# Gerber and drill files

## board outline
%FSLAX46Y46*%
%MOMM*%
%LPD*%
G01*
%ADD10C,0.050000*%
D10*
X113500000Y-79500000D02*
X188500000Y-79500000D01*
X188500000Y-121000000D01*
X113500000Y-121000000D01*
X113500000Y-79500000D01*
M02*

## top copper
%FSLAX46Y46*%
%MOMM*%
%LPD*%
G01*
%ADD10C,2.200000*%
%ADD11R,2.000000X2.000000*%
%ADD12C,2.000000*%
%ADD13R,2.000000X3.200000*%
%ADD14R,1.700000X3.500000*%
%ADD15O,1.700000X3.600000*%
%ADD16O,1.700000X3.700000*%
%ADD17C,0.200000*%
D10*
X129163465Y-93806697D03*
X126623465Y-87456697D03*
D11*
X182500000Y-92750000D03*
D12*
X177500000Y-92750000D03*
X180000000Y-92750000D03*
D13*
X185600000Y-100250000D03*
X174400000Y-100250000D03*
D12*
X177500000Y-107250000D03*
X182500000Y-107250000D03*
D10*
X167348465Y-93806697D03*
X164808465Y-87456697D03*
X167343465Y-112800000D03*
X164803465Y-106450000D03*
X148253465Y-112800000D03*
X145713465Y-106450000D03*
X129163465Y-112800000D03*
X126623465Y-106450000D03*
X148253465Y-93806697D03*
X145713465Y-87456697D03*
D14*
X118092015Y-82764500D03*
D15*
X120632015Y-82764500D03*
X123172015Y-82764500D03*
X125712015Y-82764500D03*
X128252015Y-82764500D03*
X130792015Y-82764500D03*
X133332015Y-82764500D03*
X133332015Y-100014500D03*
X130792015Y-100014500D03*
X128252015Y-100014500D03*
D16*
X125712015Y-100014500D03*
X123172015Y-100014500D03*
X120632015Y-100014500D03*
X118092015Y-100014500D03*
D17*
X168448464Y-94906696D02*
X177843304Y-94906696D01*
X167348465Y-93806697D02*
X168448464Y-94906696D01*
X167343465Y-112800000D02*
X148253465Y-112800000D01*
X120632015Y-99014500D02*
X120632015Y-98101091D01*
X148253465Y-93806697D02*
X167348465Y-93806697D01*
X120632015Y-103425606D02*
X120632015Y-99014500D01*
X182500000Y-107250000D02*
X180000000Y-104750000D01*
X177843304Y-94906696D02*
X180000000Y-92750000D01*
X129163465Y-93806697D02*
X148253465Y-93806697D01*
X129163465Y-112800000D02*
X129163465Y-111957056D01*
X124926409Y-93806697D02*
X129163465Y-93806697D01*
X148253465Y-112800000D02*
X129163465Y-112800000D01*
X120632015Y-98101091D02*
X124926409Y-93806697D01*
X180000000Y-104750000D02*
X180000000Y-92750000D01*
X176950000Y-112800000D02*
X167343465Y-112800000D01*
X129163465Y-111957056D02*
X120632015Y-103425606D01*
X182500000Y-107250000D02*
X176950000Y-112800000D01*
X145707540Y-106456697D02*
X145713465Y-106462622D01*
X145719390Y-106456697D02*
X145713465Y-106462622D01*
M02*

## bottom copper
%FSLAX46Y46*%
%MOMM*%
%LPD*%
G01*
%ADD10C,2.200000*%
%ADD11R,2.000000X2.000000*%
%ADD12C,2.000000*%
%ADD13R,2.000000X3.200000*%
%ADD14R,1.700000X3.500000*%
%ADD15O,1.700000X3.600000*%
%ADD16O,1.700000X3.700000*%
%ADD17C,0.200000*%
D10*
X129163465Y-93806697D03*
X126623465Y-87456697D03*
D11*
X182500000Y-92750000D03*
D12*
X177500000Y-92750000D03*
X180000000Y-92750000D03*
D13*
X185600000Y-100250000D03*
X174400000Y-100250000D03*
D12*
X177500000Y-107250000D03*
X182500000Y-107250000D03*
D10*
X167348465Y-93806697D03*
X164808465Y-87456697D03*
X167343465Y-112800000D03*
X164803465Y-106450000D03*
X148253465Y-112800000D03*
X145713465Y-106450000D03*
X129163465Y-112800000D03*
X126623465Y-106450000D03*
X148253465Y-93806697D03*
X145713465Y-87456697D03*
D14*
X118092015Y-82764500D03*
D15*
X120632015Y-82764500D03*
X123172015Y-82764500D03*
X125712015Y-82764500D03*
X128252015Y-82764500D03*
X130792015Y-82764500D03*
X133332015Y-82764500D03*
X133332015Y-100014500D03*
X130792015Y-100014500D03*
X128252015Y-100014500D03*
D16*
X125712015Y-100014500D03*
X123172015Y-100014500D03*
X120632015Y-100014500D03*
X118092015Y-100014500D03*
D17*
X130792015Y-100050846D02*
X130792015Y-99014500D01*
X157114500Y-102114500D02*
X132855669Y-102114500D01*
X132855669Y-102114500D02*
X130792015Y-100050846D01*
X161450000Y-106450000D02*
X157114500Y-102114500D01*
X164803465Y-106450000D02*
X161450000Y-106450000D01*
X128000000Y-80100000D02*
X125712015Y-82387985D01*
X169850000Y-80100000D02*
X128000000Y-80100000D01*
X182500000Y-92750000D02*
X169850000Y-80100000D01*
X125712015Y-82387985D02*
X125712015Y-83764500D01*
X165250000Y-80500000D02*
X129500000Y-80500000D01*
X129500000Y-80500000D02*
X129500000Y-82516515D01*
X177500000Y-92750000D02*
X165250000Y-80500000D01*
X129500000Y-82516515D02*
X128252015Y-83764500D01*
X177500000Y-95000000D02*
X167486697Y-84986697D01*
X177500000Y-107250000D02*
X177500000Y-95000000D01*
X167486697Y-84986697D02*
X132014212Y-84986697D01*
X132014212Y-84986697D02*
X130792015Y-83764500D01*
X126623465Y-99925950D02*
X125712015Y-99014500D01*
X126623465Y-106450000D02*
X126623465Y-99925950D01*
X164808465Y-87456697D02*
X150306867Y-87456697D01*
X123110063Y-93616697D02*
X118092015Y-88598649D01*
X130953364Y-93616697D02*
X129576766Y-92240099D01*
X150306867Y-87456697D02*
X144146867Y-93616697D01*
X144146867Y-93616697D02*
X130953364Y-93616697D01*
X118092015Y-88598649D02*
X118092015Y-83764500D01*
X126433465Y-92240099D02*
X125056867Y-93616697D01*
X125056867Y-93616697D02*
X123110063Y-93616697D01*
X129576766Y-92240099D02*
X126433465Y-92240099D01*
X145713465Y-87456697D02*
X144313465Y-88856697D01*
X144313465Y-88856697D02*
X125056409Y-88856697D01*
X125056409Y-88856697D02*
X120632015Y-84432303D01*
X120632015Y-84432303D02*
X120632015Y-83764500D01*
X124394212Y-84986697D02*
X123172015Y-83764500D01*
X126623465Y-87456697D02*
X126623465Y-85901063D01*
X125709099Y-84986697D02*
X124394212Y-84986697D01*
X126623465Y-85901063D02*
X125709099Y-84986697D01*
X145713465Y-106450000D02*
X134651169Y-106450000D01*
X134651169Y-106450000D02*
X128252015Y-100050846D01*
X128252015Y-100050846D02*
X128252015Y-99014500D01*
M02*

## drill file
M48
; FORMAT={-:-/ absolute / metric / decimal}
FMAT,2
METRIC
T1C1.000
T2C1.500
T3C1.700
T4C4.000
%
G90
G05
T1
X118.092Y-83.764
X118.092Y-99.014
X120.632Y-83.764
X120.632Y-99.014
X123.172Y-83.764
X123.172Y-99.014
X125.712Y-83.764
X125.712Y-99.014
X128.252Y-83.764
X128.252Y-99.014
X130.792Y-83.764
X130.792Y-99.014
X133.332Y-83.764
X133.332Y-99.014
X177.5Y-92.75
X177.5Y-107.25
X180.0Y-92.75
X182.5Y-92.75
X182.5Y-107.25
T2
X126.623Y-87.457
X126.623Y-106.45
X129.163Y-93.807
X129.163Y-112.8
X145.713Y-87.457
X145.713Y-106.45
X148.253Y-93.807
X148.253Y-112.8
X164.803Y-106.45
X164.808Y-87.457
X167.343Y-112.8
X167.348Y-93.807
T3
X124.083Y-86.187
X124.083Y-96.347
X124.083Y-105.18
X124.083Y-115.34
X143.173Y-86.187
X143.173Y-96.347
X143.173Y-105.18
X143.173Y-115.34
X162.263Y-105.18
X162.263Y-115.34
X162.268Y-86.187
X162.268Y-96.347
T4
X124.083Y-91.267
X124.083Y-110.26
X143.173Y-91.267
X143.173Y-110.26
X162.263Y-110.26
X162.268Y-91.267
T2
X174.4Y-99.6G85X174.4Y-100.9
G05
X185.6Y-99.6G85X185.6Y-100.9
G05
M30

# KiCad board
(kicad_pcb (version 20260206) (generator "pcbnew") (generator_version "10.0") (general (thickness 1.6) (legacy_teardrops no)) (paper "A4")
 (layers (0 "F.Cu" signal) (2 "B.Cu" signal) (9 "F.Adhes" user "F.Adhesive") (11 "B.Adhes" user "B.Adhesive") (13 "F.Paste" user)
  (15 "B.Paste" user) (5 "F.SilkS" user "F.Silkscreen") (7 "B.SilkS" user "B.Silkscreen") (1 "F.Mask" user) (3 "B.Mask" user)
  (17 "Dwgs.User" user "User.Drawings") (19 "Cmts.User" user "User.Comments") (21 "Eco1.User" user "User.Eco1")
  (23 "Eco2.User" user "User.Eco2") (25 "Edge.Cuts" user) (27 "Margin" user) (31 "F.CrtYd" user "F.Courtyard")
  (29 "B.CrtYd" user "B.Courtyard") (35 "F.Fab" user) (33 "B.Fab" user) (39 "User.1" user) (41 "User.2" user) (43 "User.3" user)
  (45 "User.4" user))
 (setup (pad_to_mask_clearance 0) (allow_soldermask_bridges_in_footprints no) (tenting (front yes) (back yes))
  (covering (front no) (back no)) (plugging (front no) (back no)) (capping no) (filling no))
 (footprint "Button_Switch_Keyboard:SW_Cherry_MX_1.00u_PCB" (layer "F.Cu") (at 129.163465 93.806697 -90)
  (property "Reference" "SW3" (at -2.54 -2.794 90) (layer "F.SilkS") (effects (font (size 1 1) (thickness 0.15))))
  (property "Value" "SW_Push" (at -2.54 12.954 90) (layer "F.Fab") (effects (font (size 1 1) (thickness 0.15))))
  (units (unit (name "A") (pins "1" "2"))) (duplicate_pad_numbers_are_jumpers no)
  (pad "" np_thru_hole circle (at -7.62 5.08 270) (size 1.7 1.7) (drill 1.7) (layers "*.Cu" "*.Mask"))
  (pad "" np_thru_hole circle (at -2.54 5.08 270) (size 4 4) (drill 4) (layers "*.Cu" "*.Mask"))
  (pad "" np_thru_hole circle (at 2.54 5.08 270) (size 1.7 1.7) (drill 1.7) (layers "*.Cu" "*.Mask"))
  (pad "1" thru_hole circle (at 0 0 270) (size 2.2 2.2) (drill 1.5) (layers "*.Cu" "*.Mask") (remove_unused_layers no) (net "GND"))
  (pad "2" thru_hole circle (at -6.35 2.54 270) (size 2.2 2.2) (drill 1.5) (layers "*.Cu" "*.Mask") (remove_unused_layers no)
   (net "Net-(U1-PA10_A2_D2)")))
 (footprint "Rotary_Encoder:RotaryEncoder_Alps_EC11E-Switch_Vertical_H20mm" (layer "F.Cu") (at 182.5 92.75 -90)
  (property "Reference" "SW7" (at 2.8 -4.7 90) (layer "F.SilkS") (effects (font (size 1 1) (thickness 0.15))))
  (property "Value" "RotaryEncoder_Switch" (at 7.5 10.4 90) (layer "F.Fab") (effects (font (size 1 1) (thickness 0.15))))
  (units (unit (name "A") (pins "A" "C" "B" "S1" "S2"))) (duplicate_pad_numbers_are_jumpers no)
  (pad "A" thru_hole rect (at 0 0 270) (size 2 2) (drill 1) (layers "*.Cu" "*.Mask") (remove_unused_layers no) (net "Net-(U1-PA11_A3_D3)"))
  (pad "B" thru_hole circle (at 0 5 270) (size 2 2) (drill 1) (layers "*.Cu" "*.Mask") (remove_unused_layers no)
   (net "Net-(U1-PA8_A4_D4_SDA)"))
  (pad "C" thru_hole circle (at 0 2.5 270) (size 2 2) (drill 1) (layers "*.Cu" "*.Mask") (remove_unused_layers no) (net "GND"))
  (pad "MP" thru_hole rect (at 7.5 -3.1 270) (size 3.2 2) (drill oval 2.8 1.5) (layers "*.Cu" "*.Mask") (remove_unused_layers no))
  (pad "MP" thru_hole rect (at 7.5 8.1 270) (size 3.2 2) (drill oval 2.8 1.5) (layers "*.Cu" "*.Mask") (remove_unused_layers no))
  (pad "S1" thru_hole circle (at 14.5 5 270) (size 2 2) (drill 1) (layers "*.Cu" "*.Mask") (remove_unused_layers no)
   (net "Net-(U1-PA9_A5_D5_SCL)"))
  (pad "S2" thru_hole circle (at 14.5 0 270) (size 2 2) (drill 1) (layers "*.Cu" "*.Mask") (remove_unused_layers no) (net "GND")))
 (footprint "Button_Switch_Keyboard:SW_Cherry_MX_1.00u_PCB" (layer "F.Cu") (at 167.348465 93.806697 -90)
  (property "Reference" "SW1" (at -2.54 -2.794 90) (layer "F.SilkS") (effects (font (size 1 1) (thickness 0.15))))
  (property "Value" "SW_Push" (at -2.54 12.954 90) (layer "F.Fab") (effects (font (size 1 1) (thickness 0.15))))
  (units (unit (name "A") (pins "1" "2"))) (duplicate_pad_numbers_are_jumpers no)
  (pad "" np_thru_hole circle (at -7.62 5.08 270) (size 1.7 1.7) (drill 1.7) (layers "*.Cu" "*.Mask"))
  (pad "" np_thru_hole circle (at -2.54 5.08 270) (size 4 4) (drill 4) (layers "*.Cu" "*.Mask"))
  (pad "" np_thru_hole circle (at 2.54 5.08 270) (size 1.7 1.7) (drill 1.7) (layers "*.Cu" "*.Mask"))
  (pad "1" thru_hole circle (at 0 0 270) (size 2.2 2.2) (drill 1.5) (layers "*.Cu" "*.Mask") (remove_unused_layers no) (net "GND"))
  (pad "2" thru_hole circle (at -6.35 2.54 270) (size 2.2 2.2) (drill 1.5) (layers "*.Cu" "*.Mask") (remove_unused_layers no)
   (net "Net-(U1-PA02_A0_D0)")))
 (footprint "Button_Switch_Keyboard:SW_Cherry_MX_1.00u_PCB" (layer "F.Cu") (at 167.343465 112.8 -90)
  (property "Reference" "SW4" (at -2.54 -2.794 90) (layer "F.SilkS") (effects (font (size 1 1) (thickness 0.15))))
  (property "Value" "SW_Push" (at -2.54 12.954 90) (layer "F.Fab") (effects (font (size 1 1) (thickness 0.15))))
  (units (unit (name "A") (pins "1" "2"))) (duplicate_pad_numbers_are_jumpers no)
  (pad "" np_thru_hole circle (at -7.62 5.08 270) (size 1.7 1.7) (drill 1.7) (layers "*.Cu" "*.Mask"))
  (pad "" np_thru_hole circle (at -2.54 5.08 270) (size 4 4) (drill 4) (layers "*.Cu" "*.Mask"))
  (pad "" np_thru_hole circle (at 2.54 5.08 270) (size 1.7 1.7) (drill 1.7) (layers "*.Cu" "*.Mask"))
  (pad "1" thru_hole circle (at 0 0 270) (size 2.2 2.2) (drill 1.5) (layers "*.Cu" "*.Mask") (remove_unused_layers no) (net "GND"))
  (pad "2" thru_hole circle (at -6.35 2.54 270) (size 2.2 2.2) (drill 1.5) (layers "*.Cu" "*.Mask") (remove_unused_layers no)
   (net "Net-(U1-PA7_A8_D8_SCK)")))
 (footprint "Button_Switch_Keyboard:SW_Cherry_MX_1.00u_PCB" (layer "F.Cu") (at 148.253465 112.8 -90)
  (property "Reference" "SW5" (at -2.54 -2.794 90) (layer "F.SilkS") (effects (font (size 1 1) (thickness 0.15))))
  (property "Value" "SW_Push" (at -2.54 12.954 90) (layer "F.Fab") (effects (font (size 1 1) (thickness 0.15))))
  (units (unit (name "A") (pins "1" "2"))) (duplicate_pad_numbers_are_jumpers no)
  (pad "" np_thru_hole circle (at -7.62 5.08 270) (size 1.7 1.7) (drill 1.7) (layers "*.Cu" "*.Mask"))
  (pad "" np_thru_hole circle (at -2.54 5.08 270) (size 4 4) (drill 4) (layers "*.Cu" "*.Mask"))
  (pad "" np_thru_hole circle (at 2.54 5.08 270) (size 1.7 1.7) (drill 1.7) (layers "*.Cu" "*.Mask"))
  (pad "1" thru_hole circle (at 0 0 270) (size 2.2 2.2) (drill 1.5) (layers "*.Cu" "*.Mask") (remove_unused_layers no) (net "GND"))
  (pad "2" thru_hole circle (at -6.35 2.54 270) (size 2.2 2.2) (drill 1.5) (layers "*.Cu" "*.Mask") (remove_unused_layers no)
   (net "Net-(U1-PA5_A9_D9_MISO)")))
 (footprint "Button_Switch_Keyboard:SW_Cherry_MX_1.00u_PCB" (layer "F.Cu") (at 129.163465 112.8 -90)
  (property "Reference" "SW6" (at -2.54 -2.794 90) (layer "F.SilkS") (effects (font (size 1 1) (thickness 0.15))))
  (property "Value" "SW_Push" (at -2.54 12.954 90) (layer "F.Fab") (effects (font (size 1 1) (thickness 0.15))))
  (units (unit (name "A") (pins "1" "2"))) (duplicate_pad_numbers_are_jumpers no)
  (pad "" np_thru_hole circle (at -7.62 5.08 270) (size 1.7 1.7) (drill 1.7) (layers "*.Cu" "*.Mask"))
  (pad "" np_thru_hole circle (at -2.54 5.08 270) (size 4 4) (drill 4) (layers "*.Cu" "*.Mask"))
  (pad "" np_thru_hole circle (at 2.54 5.08 270) (size 1.7 1.7) (drill 1.7) (layers "*.Cu" "*.Mask"))
  (pad "1" thru_hole circle (at 0 0 270) (size 2.2 2.2) (drill 1.5) (layers "*.Cu" "*.Mask") (remove_unused_layers no) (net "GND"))
  (pad "2" thru_hole circle (at -6.35 2.54 270) (size 2.2 2.2) (drill 1.5) (layers "*.Cu" "*.Mask") (remove_unused_layers no)
   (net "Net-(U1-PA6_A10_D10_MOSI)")))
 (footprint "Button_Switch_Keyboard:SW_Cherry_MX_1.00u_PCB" (layer "F.Cu") (at 148.253465 93.806697 -90)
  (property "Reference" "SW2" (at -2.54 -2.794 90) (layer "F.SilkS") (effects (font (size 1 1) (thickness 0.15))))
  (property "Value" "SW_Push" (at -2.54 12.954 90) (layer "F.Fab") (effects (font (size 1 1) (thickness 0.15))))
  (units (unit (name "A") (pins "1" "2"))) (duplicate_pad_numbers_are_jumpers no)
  (pad "" np_thru_hole circle (at -7.62 5.08 270) (size 1.7 1.7) (drill 1.7) (layers "*.Cu" "*.Mask"))
  (pad "" np_thru_hole circle (at -2.54 5.08 270) (size 4 4) (drill 4) (layers "*.Cu" "*.Mask"))
  (pad "" np_thru_hole circle (at 2.54 5.08 270) (size 1.7 1.7) (drill 1.7) (layers "*.Cu" "*.Mask"))
  (pad "1" thru_hole circle (at 0 0 270) (size 2.2 2.2) (drill 1.5) (layers "*.Cu" "*.Mask") (remove_unused_layers no) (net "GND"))
  (pad "2" thru_hole circle (at -6.35 2.54 270) (size 2.2 2.2) (drill 1.5) (layers "*.Cu" "*.Mask") (remove_unused_layers no)
   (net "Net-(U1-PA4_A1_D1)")))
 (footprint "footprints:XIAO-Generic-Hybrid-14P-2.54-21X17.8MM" (layer "B.Cu") (at 125.712015 91.3895 -90)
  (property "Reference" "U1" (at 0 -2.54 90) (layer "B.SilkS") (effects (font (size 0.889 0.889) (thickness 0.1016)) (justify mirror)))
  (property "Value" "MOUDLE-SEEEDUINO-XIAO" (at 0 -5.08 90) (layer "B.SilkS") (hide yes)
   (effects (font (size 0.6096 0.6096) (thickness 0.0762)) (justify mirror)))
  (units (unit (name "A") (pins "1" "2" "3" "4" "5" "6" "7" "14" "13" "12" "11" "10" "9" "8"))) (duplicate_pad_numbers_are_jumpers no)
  (pad "1" thru_hole rect (at -7.625 7.62 270) (size 3.5 1.7) (drill 1 (offset -1 0)) (layers "*.Cu" "*.Mask") (remove_unused_layers no)
   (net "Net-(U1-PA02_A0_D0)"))
  (pad "2" thru_hole oval (at -7.625 5.08 270) (size 3.6 1.7) (drill 1 (offset -1 0)) (layers "*.Cu" "*.Mask") (remove_unused_layers no)
   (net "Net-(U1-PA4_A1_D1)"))
  (pad "3" thru_hole oval (at -7.625 2.54 270) (size 3.6 1.7) (drill 1 (offset -1 0)) (layers "*.Cu" "*.Mask") (remove_unused_layers no)
   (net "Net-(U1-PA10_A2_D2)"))
  (pad "4" thru_hole oval (at -7.625 0 270) (size 3.6 1.7) (drill 1 (offset -1 0)) (layers "*.Cu" "*.Mask") (remove_unused_layers no)
   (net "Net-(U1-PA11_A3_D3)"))
  (pad "5" thru_hole oval (at -7.625 -2.54 270) (size 3.6 1.7) (drill 1 (offset -1 0)) (layers "*.Cu" "*.Mask") (remove_unused_layers no)
   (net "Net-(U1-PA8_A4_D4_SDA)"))
  (pad "6" thru_hole oval (at -7.625 -5.08 90) (size 3.6 1.7) (drill 1 (offset 1 0)) (layers "*.Cu" "*.Mask") (remove_unused_layers no)
   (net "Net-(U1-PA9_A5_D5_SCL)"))
  (pad "7" thru_hole oval (at -7.625 -7.62 270) (size 3.6 1.7) (drill 1 (offset -1 0)) (layers "*.Cu" "*.Mask") (remove_unused_layers no)
   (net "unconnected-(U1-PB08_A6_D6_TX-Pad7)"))
  (pad "8" thru_hole oval (at 7.625 -7.62 270) (size 3.6 1.7) (drill 1 (offset 1 0)) (layers "*.Cu" "*.Mask") (remove_unused_layers no)
   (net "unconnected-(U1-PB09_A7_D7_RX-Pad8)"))
  (pad "9" thru_hole oval (at 7.625 -5.08 270) (size 3.6 1.7) (drill 1 (offset 1 0)) (layers "*.Cu" "*.Mask") (remove_unused_layers no)
   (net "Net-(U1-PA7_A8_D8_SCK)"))
  (pad "10" thru_hole oval (at 7.625 -2.54 270) (size 3.6 1.7) (drill 1 (offset 1 0)) (layers "*.Cu" "*.Mask") (remove_unused_layers no)
   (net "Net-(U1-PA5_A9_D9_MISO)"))
  (pad "11" thru_hole oval (at 7.625 0 270) (size 3.7 1.7) (drill 1 (offset 1 0)) (layers "*.Cu" "*.Mask") (remove_unused_layers no)
   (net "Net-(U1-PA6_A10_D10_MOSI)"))
  (pad "12" thru_hole oval (at 7.625 2.54 270) (size 3.7 1.7) (drill 1 (offset 1 0)) (layers "*.Cu" "*.Mask") (remove_unused_layers no)
   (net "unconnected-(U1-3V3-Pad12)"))
  (pad "13" thru_hole oval (at 7.625 5.08 270) (size 3.7 1.7) (drill 1 (offset 1 0)) (layers "*.Cu" "*.Mask") (remove_unused_layers no)
   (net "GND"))
  (pad "14" thru_hole oval (at 7.625 7.62 270) (size 3.7 1.7) (drill 1 (offset 1 0)) (layers "*.Cu" "*.Mask") (remove_unused_layers no)
   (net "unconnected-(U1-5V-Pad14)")))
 (gr_rect (start 113.5 79.5) (end 188.5 121) (stroke (width 0.05) (type default)) (fill no) (layer "Edge.Cuts"))
 (segment (start 130.792015 100.050846) (end 130.792015 99.0145) (width 0.2) (layer "B.Cu") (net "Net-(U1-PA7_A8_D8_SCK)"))
 (segment (start 157.1145 102.1145) (end 132.855669 102.1145) (width 0.2) (layer "B.Cu") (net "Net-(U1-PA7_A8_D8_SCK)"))
 (segment (start 132.855669 102.1145) (end 130.792015 100.050846) (width 0.2) (layer "B.Cu") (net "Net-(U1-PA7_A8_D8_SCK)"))
 (segment (start 161.45 106.45) (end 157.1145 102.1145) (width 0.2) (layer "B.Cu") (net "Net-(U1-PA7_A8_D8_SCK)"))
 (segment (start 164.803465 106.45) (end 161.45 106.45) (width 0.2) (layer "B.Cu") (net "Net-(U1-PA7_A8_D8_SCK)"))
 (segment (start 168.448464 94.906696) (end 177.843304 94.906696) (width 0.2) (layer "F.Cu") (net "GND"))
 (segment (start 167.348465 93.806697) (end 168.448464 94.906696) (width 0.2) (layer "F.Cu") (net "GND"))
 (segment (start 167.343465 112.8) (end 148.253465 112.8) (width 0.2) (layer "F.Cu") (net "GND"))
 (segment (start 120.632015 99.0145) (end 120.632015 98.101091) (width 0.2) (layer "F.Cu") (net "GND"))
 (segment (start 148.253465 93.806697) (end 167.348465 93.806697) (width 0.2) (layer "F.Cu") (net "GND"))
 (segment (start 120.632015 103.425606) (end 120.632015 99.0145) (width 0.2) (layer "F.Cu") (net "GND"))
 (segment (start 182.5 107.25) (end 180 104.75) (width 0.2) (layer "F.Cu") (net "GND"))
 (segment (start 177.843304 94.906696) (end 180 92.75) (width 0.2) (layer "F.Cu") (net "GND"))
 (segment (start 129.163465 93.806697) (end 148.253465 93.806697) (width 0.2) (layer "F.Cu") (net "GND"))
 (segment (start 129.163465 112.8) (end 129.163465 111.957056) (width 0.2) (layer "F.Cu") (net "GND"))
 (segment (start 124.926409 93.806697) (end 129.163465 93.806697) (width 0.2) (layer "F.Cu") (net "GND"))
 (segment (start 148.253465 112.8) (end 129.163465 112.8) (width 0.2) (layer "F.Cu") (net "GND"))
 (segment (start 120.632015 98.101091) (end 124.926409 93.806697) (width 0.2) (layer "F.Cu") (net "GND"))
 (segment (start 180 104.75) (end 180 92.75) (width 0.2) (layer "F.Cu") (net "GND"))
 (segment (start 176.95 112.8) (end 167.343465 112.8) (width 0.2) (layer "F.Cu") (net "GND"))
 (segment (start 129.163465 111.957056) (end 120.632015 103.425606) (width 0.2) (layer "F.Cu") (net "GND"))
 (segment (start 182.5 107.25) (end 176.95 112.8) (width 0.2) (layer "F.Cu") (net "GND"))
 (segment (start 128 80.1) (end 125.712015 82.387985) (width 0.2) (layer "B.Cu") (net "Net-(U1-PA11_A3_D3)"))
 (segment (start 169.85 80.1) (end 128 80.1) (width 0.2) (layer "B.Cu") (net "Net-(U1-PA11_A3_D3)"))
 (segment (start 182.5 92.75) (end 169.85 80.1) (width 0.2) (layer "B.Cu") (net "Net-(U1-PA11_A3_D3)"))
 (segment (start 125.712015 82.387985) (end 125.712015 83.7645) (width 0.2) (layer "B.Cu") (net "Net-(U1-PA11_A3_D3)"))
 (segment (start 165.25 80.5) (end 129.5 80.5) (width 0.2) (layer "B.Cu") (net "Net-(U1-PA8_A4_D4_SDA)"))
 (segment (start 129.5 80.5) (end 129.5 82.516515) (width 0.2) (layer "B.Cu") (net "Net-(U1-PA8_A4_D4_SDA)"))
 (segment (start 177.5 92.75) (end 165.25 80.5) (width 0.2) (layer "B.Cu") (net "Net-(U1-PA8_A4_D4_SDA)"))
 (segment (start 129.5 82.516515) (end 128.252015 83.7645) (width 0.2) (layer "B.Cu") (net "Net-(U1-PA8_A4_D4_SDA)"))
 (segment (start 177.5 95) (end 167.486697 84.986697) (width 0.2) (layer "B.Cu") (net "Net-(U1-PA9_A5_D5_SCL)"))
 (segment (start 177.5 107.25) (end 177.5 95) (width 0.2) (layer "B.Cu") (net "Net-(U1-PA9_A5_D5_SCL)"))
 (segment (start 167.486697 84.986697) (end 132.014212 84.986697) (width 0.2) (layer "B.Cu") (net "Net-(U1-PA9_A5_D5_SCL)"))
 (segment (start 132.014212 84.986697) (end 130.792015 83.7645) (width 0.2) (layer "B.Cu") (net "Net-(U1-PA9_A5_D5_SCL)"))
 (segment (start 126.623465 99.92595) (end 125.712015 99.0145) (width 0.2) (layer "B.Cu") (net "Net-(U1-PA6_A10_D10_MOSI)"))
 (segment (start 126.623465 106.45) (end 126.623465 99.92595) (width 0.2) (layer "B.Cu") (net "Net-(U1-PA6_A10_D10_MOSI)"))
 (segment (start 164.808465 87.456697) (end 150.306867 87.456697) (width 0.2) (layer "B.Cu") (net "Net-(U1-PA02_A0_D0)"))
 (segment (start 123.110063 93.616697) (end 118.092015 88.598649) (width 0.2) (layer "B.Cu") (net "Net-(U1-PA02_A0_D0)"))
 (segment (start 130.953364 93.616697) (end 129.576766 92.240099) (width 0.2) (layer "B.Cu") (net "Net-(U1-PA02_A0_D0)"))
 (segment (start 150.306867 87.456697) (end 144.146867 93.616697) (width 0.2) (layer "B.Cu") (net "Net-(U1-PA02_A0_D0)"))
 (segment (start 144.146867 93.616697) (end 130.953364 93.616697) (width 0.2) (layer "B.Cu") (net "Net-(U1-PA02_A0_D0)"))
 (segment (start 118.092015 88.598649) (end 118.092015 83.7645) (width 0.2) (layer "B.Cu") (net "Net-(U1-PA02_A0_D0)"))
 (segment (start 126.433465 92.240099) (end 125.056867 93.616697) (width 0.2) (layer "B.Cu") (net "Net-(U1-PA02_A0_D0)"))
 (segment (start 125.056867 93.616697) (end 123.110063 93.616697) (width 0.2) (layer "B.Cu") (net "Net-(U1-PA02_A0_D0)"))
 (segment (start 129.576766 92.240099) (end 126.433465 92.240099) (width 0.2) (layer "B.Cu") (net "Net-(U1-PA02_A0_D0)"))
 (segment (start 145.713465 87.456697) (end 144.313465 88.856697) (width 0.2) (layer "B.Cu") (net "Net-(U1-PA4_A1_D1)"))
 (segment (start 144.313465 88.856697) (end 125.056409 88.856697) (width 0.2) (layer "B.Cu") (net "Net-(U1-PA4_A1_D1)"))
 (segment (start 125.056409 88.856697) (end 120.632015 84.432303) (width 0.2) (layer "B.Cu") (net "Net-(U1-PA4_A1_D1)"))
 (segment (start 120.632015 84.432303) (end 120.632015 83.7645) (width 0.2) (layer "B.Cu") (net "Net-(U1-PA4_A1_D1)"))
 (segment (start 124.394212 84.986697) (end 123.172015 83.7645) (width 0.2) (layer "B.Cu") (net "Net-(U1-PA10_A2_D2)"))
 (segment (start 126.623465 87.456697) (end 126.623465 85.901063) (width 0.2) (layer "B.Cu") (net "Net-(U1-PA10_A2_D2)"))
 (segment (start 125.709099 84.986697) (end 124.394212 84.986697) (width 0.2) (layer "B.Cu") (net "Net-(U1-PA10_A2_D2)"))
 (segment (start 126.623465 85.901063) (end 125.709099 84.986697) (width 0.2) (layer "B.Cu") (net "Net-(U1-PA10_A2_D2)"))
 (segment (start 145.70754 106.456697) (end 145.713465 106.462622) (width 0.2) (layer "F.Cu") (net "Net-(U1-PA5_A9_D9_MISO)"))
 (segment (start 145.71939 106.456697) (end 145.713465 106.462622) (width 0.2) (layer "F.Cu") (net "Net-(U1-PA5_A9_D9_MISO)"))
 (segment (start 145.713465 106.45) (end 134.651169 106.45) (width 0.2) (layer "B.Cu") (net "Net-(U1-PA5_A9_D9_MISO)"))
 (segment (start 134.651169 106.45) (end 128.252015 100.050846) (width 0.2) (layer "B.Cu") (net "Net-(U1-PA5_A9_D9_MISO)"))
 (segment (start 128.252015 100.050846) (end 128.252015 99.0145) (width 0.2) (layer "B.Cu") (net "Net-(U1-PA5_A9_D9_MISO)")))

